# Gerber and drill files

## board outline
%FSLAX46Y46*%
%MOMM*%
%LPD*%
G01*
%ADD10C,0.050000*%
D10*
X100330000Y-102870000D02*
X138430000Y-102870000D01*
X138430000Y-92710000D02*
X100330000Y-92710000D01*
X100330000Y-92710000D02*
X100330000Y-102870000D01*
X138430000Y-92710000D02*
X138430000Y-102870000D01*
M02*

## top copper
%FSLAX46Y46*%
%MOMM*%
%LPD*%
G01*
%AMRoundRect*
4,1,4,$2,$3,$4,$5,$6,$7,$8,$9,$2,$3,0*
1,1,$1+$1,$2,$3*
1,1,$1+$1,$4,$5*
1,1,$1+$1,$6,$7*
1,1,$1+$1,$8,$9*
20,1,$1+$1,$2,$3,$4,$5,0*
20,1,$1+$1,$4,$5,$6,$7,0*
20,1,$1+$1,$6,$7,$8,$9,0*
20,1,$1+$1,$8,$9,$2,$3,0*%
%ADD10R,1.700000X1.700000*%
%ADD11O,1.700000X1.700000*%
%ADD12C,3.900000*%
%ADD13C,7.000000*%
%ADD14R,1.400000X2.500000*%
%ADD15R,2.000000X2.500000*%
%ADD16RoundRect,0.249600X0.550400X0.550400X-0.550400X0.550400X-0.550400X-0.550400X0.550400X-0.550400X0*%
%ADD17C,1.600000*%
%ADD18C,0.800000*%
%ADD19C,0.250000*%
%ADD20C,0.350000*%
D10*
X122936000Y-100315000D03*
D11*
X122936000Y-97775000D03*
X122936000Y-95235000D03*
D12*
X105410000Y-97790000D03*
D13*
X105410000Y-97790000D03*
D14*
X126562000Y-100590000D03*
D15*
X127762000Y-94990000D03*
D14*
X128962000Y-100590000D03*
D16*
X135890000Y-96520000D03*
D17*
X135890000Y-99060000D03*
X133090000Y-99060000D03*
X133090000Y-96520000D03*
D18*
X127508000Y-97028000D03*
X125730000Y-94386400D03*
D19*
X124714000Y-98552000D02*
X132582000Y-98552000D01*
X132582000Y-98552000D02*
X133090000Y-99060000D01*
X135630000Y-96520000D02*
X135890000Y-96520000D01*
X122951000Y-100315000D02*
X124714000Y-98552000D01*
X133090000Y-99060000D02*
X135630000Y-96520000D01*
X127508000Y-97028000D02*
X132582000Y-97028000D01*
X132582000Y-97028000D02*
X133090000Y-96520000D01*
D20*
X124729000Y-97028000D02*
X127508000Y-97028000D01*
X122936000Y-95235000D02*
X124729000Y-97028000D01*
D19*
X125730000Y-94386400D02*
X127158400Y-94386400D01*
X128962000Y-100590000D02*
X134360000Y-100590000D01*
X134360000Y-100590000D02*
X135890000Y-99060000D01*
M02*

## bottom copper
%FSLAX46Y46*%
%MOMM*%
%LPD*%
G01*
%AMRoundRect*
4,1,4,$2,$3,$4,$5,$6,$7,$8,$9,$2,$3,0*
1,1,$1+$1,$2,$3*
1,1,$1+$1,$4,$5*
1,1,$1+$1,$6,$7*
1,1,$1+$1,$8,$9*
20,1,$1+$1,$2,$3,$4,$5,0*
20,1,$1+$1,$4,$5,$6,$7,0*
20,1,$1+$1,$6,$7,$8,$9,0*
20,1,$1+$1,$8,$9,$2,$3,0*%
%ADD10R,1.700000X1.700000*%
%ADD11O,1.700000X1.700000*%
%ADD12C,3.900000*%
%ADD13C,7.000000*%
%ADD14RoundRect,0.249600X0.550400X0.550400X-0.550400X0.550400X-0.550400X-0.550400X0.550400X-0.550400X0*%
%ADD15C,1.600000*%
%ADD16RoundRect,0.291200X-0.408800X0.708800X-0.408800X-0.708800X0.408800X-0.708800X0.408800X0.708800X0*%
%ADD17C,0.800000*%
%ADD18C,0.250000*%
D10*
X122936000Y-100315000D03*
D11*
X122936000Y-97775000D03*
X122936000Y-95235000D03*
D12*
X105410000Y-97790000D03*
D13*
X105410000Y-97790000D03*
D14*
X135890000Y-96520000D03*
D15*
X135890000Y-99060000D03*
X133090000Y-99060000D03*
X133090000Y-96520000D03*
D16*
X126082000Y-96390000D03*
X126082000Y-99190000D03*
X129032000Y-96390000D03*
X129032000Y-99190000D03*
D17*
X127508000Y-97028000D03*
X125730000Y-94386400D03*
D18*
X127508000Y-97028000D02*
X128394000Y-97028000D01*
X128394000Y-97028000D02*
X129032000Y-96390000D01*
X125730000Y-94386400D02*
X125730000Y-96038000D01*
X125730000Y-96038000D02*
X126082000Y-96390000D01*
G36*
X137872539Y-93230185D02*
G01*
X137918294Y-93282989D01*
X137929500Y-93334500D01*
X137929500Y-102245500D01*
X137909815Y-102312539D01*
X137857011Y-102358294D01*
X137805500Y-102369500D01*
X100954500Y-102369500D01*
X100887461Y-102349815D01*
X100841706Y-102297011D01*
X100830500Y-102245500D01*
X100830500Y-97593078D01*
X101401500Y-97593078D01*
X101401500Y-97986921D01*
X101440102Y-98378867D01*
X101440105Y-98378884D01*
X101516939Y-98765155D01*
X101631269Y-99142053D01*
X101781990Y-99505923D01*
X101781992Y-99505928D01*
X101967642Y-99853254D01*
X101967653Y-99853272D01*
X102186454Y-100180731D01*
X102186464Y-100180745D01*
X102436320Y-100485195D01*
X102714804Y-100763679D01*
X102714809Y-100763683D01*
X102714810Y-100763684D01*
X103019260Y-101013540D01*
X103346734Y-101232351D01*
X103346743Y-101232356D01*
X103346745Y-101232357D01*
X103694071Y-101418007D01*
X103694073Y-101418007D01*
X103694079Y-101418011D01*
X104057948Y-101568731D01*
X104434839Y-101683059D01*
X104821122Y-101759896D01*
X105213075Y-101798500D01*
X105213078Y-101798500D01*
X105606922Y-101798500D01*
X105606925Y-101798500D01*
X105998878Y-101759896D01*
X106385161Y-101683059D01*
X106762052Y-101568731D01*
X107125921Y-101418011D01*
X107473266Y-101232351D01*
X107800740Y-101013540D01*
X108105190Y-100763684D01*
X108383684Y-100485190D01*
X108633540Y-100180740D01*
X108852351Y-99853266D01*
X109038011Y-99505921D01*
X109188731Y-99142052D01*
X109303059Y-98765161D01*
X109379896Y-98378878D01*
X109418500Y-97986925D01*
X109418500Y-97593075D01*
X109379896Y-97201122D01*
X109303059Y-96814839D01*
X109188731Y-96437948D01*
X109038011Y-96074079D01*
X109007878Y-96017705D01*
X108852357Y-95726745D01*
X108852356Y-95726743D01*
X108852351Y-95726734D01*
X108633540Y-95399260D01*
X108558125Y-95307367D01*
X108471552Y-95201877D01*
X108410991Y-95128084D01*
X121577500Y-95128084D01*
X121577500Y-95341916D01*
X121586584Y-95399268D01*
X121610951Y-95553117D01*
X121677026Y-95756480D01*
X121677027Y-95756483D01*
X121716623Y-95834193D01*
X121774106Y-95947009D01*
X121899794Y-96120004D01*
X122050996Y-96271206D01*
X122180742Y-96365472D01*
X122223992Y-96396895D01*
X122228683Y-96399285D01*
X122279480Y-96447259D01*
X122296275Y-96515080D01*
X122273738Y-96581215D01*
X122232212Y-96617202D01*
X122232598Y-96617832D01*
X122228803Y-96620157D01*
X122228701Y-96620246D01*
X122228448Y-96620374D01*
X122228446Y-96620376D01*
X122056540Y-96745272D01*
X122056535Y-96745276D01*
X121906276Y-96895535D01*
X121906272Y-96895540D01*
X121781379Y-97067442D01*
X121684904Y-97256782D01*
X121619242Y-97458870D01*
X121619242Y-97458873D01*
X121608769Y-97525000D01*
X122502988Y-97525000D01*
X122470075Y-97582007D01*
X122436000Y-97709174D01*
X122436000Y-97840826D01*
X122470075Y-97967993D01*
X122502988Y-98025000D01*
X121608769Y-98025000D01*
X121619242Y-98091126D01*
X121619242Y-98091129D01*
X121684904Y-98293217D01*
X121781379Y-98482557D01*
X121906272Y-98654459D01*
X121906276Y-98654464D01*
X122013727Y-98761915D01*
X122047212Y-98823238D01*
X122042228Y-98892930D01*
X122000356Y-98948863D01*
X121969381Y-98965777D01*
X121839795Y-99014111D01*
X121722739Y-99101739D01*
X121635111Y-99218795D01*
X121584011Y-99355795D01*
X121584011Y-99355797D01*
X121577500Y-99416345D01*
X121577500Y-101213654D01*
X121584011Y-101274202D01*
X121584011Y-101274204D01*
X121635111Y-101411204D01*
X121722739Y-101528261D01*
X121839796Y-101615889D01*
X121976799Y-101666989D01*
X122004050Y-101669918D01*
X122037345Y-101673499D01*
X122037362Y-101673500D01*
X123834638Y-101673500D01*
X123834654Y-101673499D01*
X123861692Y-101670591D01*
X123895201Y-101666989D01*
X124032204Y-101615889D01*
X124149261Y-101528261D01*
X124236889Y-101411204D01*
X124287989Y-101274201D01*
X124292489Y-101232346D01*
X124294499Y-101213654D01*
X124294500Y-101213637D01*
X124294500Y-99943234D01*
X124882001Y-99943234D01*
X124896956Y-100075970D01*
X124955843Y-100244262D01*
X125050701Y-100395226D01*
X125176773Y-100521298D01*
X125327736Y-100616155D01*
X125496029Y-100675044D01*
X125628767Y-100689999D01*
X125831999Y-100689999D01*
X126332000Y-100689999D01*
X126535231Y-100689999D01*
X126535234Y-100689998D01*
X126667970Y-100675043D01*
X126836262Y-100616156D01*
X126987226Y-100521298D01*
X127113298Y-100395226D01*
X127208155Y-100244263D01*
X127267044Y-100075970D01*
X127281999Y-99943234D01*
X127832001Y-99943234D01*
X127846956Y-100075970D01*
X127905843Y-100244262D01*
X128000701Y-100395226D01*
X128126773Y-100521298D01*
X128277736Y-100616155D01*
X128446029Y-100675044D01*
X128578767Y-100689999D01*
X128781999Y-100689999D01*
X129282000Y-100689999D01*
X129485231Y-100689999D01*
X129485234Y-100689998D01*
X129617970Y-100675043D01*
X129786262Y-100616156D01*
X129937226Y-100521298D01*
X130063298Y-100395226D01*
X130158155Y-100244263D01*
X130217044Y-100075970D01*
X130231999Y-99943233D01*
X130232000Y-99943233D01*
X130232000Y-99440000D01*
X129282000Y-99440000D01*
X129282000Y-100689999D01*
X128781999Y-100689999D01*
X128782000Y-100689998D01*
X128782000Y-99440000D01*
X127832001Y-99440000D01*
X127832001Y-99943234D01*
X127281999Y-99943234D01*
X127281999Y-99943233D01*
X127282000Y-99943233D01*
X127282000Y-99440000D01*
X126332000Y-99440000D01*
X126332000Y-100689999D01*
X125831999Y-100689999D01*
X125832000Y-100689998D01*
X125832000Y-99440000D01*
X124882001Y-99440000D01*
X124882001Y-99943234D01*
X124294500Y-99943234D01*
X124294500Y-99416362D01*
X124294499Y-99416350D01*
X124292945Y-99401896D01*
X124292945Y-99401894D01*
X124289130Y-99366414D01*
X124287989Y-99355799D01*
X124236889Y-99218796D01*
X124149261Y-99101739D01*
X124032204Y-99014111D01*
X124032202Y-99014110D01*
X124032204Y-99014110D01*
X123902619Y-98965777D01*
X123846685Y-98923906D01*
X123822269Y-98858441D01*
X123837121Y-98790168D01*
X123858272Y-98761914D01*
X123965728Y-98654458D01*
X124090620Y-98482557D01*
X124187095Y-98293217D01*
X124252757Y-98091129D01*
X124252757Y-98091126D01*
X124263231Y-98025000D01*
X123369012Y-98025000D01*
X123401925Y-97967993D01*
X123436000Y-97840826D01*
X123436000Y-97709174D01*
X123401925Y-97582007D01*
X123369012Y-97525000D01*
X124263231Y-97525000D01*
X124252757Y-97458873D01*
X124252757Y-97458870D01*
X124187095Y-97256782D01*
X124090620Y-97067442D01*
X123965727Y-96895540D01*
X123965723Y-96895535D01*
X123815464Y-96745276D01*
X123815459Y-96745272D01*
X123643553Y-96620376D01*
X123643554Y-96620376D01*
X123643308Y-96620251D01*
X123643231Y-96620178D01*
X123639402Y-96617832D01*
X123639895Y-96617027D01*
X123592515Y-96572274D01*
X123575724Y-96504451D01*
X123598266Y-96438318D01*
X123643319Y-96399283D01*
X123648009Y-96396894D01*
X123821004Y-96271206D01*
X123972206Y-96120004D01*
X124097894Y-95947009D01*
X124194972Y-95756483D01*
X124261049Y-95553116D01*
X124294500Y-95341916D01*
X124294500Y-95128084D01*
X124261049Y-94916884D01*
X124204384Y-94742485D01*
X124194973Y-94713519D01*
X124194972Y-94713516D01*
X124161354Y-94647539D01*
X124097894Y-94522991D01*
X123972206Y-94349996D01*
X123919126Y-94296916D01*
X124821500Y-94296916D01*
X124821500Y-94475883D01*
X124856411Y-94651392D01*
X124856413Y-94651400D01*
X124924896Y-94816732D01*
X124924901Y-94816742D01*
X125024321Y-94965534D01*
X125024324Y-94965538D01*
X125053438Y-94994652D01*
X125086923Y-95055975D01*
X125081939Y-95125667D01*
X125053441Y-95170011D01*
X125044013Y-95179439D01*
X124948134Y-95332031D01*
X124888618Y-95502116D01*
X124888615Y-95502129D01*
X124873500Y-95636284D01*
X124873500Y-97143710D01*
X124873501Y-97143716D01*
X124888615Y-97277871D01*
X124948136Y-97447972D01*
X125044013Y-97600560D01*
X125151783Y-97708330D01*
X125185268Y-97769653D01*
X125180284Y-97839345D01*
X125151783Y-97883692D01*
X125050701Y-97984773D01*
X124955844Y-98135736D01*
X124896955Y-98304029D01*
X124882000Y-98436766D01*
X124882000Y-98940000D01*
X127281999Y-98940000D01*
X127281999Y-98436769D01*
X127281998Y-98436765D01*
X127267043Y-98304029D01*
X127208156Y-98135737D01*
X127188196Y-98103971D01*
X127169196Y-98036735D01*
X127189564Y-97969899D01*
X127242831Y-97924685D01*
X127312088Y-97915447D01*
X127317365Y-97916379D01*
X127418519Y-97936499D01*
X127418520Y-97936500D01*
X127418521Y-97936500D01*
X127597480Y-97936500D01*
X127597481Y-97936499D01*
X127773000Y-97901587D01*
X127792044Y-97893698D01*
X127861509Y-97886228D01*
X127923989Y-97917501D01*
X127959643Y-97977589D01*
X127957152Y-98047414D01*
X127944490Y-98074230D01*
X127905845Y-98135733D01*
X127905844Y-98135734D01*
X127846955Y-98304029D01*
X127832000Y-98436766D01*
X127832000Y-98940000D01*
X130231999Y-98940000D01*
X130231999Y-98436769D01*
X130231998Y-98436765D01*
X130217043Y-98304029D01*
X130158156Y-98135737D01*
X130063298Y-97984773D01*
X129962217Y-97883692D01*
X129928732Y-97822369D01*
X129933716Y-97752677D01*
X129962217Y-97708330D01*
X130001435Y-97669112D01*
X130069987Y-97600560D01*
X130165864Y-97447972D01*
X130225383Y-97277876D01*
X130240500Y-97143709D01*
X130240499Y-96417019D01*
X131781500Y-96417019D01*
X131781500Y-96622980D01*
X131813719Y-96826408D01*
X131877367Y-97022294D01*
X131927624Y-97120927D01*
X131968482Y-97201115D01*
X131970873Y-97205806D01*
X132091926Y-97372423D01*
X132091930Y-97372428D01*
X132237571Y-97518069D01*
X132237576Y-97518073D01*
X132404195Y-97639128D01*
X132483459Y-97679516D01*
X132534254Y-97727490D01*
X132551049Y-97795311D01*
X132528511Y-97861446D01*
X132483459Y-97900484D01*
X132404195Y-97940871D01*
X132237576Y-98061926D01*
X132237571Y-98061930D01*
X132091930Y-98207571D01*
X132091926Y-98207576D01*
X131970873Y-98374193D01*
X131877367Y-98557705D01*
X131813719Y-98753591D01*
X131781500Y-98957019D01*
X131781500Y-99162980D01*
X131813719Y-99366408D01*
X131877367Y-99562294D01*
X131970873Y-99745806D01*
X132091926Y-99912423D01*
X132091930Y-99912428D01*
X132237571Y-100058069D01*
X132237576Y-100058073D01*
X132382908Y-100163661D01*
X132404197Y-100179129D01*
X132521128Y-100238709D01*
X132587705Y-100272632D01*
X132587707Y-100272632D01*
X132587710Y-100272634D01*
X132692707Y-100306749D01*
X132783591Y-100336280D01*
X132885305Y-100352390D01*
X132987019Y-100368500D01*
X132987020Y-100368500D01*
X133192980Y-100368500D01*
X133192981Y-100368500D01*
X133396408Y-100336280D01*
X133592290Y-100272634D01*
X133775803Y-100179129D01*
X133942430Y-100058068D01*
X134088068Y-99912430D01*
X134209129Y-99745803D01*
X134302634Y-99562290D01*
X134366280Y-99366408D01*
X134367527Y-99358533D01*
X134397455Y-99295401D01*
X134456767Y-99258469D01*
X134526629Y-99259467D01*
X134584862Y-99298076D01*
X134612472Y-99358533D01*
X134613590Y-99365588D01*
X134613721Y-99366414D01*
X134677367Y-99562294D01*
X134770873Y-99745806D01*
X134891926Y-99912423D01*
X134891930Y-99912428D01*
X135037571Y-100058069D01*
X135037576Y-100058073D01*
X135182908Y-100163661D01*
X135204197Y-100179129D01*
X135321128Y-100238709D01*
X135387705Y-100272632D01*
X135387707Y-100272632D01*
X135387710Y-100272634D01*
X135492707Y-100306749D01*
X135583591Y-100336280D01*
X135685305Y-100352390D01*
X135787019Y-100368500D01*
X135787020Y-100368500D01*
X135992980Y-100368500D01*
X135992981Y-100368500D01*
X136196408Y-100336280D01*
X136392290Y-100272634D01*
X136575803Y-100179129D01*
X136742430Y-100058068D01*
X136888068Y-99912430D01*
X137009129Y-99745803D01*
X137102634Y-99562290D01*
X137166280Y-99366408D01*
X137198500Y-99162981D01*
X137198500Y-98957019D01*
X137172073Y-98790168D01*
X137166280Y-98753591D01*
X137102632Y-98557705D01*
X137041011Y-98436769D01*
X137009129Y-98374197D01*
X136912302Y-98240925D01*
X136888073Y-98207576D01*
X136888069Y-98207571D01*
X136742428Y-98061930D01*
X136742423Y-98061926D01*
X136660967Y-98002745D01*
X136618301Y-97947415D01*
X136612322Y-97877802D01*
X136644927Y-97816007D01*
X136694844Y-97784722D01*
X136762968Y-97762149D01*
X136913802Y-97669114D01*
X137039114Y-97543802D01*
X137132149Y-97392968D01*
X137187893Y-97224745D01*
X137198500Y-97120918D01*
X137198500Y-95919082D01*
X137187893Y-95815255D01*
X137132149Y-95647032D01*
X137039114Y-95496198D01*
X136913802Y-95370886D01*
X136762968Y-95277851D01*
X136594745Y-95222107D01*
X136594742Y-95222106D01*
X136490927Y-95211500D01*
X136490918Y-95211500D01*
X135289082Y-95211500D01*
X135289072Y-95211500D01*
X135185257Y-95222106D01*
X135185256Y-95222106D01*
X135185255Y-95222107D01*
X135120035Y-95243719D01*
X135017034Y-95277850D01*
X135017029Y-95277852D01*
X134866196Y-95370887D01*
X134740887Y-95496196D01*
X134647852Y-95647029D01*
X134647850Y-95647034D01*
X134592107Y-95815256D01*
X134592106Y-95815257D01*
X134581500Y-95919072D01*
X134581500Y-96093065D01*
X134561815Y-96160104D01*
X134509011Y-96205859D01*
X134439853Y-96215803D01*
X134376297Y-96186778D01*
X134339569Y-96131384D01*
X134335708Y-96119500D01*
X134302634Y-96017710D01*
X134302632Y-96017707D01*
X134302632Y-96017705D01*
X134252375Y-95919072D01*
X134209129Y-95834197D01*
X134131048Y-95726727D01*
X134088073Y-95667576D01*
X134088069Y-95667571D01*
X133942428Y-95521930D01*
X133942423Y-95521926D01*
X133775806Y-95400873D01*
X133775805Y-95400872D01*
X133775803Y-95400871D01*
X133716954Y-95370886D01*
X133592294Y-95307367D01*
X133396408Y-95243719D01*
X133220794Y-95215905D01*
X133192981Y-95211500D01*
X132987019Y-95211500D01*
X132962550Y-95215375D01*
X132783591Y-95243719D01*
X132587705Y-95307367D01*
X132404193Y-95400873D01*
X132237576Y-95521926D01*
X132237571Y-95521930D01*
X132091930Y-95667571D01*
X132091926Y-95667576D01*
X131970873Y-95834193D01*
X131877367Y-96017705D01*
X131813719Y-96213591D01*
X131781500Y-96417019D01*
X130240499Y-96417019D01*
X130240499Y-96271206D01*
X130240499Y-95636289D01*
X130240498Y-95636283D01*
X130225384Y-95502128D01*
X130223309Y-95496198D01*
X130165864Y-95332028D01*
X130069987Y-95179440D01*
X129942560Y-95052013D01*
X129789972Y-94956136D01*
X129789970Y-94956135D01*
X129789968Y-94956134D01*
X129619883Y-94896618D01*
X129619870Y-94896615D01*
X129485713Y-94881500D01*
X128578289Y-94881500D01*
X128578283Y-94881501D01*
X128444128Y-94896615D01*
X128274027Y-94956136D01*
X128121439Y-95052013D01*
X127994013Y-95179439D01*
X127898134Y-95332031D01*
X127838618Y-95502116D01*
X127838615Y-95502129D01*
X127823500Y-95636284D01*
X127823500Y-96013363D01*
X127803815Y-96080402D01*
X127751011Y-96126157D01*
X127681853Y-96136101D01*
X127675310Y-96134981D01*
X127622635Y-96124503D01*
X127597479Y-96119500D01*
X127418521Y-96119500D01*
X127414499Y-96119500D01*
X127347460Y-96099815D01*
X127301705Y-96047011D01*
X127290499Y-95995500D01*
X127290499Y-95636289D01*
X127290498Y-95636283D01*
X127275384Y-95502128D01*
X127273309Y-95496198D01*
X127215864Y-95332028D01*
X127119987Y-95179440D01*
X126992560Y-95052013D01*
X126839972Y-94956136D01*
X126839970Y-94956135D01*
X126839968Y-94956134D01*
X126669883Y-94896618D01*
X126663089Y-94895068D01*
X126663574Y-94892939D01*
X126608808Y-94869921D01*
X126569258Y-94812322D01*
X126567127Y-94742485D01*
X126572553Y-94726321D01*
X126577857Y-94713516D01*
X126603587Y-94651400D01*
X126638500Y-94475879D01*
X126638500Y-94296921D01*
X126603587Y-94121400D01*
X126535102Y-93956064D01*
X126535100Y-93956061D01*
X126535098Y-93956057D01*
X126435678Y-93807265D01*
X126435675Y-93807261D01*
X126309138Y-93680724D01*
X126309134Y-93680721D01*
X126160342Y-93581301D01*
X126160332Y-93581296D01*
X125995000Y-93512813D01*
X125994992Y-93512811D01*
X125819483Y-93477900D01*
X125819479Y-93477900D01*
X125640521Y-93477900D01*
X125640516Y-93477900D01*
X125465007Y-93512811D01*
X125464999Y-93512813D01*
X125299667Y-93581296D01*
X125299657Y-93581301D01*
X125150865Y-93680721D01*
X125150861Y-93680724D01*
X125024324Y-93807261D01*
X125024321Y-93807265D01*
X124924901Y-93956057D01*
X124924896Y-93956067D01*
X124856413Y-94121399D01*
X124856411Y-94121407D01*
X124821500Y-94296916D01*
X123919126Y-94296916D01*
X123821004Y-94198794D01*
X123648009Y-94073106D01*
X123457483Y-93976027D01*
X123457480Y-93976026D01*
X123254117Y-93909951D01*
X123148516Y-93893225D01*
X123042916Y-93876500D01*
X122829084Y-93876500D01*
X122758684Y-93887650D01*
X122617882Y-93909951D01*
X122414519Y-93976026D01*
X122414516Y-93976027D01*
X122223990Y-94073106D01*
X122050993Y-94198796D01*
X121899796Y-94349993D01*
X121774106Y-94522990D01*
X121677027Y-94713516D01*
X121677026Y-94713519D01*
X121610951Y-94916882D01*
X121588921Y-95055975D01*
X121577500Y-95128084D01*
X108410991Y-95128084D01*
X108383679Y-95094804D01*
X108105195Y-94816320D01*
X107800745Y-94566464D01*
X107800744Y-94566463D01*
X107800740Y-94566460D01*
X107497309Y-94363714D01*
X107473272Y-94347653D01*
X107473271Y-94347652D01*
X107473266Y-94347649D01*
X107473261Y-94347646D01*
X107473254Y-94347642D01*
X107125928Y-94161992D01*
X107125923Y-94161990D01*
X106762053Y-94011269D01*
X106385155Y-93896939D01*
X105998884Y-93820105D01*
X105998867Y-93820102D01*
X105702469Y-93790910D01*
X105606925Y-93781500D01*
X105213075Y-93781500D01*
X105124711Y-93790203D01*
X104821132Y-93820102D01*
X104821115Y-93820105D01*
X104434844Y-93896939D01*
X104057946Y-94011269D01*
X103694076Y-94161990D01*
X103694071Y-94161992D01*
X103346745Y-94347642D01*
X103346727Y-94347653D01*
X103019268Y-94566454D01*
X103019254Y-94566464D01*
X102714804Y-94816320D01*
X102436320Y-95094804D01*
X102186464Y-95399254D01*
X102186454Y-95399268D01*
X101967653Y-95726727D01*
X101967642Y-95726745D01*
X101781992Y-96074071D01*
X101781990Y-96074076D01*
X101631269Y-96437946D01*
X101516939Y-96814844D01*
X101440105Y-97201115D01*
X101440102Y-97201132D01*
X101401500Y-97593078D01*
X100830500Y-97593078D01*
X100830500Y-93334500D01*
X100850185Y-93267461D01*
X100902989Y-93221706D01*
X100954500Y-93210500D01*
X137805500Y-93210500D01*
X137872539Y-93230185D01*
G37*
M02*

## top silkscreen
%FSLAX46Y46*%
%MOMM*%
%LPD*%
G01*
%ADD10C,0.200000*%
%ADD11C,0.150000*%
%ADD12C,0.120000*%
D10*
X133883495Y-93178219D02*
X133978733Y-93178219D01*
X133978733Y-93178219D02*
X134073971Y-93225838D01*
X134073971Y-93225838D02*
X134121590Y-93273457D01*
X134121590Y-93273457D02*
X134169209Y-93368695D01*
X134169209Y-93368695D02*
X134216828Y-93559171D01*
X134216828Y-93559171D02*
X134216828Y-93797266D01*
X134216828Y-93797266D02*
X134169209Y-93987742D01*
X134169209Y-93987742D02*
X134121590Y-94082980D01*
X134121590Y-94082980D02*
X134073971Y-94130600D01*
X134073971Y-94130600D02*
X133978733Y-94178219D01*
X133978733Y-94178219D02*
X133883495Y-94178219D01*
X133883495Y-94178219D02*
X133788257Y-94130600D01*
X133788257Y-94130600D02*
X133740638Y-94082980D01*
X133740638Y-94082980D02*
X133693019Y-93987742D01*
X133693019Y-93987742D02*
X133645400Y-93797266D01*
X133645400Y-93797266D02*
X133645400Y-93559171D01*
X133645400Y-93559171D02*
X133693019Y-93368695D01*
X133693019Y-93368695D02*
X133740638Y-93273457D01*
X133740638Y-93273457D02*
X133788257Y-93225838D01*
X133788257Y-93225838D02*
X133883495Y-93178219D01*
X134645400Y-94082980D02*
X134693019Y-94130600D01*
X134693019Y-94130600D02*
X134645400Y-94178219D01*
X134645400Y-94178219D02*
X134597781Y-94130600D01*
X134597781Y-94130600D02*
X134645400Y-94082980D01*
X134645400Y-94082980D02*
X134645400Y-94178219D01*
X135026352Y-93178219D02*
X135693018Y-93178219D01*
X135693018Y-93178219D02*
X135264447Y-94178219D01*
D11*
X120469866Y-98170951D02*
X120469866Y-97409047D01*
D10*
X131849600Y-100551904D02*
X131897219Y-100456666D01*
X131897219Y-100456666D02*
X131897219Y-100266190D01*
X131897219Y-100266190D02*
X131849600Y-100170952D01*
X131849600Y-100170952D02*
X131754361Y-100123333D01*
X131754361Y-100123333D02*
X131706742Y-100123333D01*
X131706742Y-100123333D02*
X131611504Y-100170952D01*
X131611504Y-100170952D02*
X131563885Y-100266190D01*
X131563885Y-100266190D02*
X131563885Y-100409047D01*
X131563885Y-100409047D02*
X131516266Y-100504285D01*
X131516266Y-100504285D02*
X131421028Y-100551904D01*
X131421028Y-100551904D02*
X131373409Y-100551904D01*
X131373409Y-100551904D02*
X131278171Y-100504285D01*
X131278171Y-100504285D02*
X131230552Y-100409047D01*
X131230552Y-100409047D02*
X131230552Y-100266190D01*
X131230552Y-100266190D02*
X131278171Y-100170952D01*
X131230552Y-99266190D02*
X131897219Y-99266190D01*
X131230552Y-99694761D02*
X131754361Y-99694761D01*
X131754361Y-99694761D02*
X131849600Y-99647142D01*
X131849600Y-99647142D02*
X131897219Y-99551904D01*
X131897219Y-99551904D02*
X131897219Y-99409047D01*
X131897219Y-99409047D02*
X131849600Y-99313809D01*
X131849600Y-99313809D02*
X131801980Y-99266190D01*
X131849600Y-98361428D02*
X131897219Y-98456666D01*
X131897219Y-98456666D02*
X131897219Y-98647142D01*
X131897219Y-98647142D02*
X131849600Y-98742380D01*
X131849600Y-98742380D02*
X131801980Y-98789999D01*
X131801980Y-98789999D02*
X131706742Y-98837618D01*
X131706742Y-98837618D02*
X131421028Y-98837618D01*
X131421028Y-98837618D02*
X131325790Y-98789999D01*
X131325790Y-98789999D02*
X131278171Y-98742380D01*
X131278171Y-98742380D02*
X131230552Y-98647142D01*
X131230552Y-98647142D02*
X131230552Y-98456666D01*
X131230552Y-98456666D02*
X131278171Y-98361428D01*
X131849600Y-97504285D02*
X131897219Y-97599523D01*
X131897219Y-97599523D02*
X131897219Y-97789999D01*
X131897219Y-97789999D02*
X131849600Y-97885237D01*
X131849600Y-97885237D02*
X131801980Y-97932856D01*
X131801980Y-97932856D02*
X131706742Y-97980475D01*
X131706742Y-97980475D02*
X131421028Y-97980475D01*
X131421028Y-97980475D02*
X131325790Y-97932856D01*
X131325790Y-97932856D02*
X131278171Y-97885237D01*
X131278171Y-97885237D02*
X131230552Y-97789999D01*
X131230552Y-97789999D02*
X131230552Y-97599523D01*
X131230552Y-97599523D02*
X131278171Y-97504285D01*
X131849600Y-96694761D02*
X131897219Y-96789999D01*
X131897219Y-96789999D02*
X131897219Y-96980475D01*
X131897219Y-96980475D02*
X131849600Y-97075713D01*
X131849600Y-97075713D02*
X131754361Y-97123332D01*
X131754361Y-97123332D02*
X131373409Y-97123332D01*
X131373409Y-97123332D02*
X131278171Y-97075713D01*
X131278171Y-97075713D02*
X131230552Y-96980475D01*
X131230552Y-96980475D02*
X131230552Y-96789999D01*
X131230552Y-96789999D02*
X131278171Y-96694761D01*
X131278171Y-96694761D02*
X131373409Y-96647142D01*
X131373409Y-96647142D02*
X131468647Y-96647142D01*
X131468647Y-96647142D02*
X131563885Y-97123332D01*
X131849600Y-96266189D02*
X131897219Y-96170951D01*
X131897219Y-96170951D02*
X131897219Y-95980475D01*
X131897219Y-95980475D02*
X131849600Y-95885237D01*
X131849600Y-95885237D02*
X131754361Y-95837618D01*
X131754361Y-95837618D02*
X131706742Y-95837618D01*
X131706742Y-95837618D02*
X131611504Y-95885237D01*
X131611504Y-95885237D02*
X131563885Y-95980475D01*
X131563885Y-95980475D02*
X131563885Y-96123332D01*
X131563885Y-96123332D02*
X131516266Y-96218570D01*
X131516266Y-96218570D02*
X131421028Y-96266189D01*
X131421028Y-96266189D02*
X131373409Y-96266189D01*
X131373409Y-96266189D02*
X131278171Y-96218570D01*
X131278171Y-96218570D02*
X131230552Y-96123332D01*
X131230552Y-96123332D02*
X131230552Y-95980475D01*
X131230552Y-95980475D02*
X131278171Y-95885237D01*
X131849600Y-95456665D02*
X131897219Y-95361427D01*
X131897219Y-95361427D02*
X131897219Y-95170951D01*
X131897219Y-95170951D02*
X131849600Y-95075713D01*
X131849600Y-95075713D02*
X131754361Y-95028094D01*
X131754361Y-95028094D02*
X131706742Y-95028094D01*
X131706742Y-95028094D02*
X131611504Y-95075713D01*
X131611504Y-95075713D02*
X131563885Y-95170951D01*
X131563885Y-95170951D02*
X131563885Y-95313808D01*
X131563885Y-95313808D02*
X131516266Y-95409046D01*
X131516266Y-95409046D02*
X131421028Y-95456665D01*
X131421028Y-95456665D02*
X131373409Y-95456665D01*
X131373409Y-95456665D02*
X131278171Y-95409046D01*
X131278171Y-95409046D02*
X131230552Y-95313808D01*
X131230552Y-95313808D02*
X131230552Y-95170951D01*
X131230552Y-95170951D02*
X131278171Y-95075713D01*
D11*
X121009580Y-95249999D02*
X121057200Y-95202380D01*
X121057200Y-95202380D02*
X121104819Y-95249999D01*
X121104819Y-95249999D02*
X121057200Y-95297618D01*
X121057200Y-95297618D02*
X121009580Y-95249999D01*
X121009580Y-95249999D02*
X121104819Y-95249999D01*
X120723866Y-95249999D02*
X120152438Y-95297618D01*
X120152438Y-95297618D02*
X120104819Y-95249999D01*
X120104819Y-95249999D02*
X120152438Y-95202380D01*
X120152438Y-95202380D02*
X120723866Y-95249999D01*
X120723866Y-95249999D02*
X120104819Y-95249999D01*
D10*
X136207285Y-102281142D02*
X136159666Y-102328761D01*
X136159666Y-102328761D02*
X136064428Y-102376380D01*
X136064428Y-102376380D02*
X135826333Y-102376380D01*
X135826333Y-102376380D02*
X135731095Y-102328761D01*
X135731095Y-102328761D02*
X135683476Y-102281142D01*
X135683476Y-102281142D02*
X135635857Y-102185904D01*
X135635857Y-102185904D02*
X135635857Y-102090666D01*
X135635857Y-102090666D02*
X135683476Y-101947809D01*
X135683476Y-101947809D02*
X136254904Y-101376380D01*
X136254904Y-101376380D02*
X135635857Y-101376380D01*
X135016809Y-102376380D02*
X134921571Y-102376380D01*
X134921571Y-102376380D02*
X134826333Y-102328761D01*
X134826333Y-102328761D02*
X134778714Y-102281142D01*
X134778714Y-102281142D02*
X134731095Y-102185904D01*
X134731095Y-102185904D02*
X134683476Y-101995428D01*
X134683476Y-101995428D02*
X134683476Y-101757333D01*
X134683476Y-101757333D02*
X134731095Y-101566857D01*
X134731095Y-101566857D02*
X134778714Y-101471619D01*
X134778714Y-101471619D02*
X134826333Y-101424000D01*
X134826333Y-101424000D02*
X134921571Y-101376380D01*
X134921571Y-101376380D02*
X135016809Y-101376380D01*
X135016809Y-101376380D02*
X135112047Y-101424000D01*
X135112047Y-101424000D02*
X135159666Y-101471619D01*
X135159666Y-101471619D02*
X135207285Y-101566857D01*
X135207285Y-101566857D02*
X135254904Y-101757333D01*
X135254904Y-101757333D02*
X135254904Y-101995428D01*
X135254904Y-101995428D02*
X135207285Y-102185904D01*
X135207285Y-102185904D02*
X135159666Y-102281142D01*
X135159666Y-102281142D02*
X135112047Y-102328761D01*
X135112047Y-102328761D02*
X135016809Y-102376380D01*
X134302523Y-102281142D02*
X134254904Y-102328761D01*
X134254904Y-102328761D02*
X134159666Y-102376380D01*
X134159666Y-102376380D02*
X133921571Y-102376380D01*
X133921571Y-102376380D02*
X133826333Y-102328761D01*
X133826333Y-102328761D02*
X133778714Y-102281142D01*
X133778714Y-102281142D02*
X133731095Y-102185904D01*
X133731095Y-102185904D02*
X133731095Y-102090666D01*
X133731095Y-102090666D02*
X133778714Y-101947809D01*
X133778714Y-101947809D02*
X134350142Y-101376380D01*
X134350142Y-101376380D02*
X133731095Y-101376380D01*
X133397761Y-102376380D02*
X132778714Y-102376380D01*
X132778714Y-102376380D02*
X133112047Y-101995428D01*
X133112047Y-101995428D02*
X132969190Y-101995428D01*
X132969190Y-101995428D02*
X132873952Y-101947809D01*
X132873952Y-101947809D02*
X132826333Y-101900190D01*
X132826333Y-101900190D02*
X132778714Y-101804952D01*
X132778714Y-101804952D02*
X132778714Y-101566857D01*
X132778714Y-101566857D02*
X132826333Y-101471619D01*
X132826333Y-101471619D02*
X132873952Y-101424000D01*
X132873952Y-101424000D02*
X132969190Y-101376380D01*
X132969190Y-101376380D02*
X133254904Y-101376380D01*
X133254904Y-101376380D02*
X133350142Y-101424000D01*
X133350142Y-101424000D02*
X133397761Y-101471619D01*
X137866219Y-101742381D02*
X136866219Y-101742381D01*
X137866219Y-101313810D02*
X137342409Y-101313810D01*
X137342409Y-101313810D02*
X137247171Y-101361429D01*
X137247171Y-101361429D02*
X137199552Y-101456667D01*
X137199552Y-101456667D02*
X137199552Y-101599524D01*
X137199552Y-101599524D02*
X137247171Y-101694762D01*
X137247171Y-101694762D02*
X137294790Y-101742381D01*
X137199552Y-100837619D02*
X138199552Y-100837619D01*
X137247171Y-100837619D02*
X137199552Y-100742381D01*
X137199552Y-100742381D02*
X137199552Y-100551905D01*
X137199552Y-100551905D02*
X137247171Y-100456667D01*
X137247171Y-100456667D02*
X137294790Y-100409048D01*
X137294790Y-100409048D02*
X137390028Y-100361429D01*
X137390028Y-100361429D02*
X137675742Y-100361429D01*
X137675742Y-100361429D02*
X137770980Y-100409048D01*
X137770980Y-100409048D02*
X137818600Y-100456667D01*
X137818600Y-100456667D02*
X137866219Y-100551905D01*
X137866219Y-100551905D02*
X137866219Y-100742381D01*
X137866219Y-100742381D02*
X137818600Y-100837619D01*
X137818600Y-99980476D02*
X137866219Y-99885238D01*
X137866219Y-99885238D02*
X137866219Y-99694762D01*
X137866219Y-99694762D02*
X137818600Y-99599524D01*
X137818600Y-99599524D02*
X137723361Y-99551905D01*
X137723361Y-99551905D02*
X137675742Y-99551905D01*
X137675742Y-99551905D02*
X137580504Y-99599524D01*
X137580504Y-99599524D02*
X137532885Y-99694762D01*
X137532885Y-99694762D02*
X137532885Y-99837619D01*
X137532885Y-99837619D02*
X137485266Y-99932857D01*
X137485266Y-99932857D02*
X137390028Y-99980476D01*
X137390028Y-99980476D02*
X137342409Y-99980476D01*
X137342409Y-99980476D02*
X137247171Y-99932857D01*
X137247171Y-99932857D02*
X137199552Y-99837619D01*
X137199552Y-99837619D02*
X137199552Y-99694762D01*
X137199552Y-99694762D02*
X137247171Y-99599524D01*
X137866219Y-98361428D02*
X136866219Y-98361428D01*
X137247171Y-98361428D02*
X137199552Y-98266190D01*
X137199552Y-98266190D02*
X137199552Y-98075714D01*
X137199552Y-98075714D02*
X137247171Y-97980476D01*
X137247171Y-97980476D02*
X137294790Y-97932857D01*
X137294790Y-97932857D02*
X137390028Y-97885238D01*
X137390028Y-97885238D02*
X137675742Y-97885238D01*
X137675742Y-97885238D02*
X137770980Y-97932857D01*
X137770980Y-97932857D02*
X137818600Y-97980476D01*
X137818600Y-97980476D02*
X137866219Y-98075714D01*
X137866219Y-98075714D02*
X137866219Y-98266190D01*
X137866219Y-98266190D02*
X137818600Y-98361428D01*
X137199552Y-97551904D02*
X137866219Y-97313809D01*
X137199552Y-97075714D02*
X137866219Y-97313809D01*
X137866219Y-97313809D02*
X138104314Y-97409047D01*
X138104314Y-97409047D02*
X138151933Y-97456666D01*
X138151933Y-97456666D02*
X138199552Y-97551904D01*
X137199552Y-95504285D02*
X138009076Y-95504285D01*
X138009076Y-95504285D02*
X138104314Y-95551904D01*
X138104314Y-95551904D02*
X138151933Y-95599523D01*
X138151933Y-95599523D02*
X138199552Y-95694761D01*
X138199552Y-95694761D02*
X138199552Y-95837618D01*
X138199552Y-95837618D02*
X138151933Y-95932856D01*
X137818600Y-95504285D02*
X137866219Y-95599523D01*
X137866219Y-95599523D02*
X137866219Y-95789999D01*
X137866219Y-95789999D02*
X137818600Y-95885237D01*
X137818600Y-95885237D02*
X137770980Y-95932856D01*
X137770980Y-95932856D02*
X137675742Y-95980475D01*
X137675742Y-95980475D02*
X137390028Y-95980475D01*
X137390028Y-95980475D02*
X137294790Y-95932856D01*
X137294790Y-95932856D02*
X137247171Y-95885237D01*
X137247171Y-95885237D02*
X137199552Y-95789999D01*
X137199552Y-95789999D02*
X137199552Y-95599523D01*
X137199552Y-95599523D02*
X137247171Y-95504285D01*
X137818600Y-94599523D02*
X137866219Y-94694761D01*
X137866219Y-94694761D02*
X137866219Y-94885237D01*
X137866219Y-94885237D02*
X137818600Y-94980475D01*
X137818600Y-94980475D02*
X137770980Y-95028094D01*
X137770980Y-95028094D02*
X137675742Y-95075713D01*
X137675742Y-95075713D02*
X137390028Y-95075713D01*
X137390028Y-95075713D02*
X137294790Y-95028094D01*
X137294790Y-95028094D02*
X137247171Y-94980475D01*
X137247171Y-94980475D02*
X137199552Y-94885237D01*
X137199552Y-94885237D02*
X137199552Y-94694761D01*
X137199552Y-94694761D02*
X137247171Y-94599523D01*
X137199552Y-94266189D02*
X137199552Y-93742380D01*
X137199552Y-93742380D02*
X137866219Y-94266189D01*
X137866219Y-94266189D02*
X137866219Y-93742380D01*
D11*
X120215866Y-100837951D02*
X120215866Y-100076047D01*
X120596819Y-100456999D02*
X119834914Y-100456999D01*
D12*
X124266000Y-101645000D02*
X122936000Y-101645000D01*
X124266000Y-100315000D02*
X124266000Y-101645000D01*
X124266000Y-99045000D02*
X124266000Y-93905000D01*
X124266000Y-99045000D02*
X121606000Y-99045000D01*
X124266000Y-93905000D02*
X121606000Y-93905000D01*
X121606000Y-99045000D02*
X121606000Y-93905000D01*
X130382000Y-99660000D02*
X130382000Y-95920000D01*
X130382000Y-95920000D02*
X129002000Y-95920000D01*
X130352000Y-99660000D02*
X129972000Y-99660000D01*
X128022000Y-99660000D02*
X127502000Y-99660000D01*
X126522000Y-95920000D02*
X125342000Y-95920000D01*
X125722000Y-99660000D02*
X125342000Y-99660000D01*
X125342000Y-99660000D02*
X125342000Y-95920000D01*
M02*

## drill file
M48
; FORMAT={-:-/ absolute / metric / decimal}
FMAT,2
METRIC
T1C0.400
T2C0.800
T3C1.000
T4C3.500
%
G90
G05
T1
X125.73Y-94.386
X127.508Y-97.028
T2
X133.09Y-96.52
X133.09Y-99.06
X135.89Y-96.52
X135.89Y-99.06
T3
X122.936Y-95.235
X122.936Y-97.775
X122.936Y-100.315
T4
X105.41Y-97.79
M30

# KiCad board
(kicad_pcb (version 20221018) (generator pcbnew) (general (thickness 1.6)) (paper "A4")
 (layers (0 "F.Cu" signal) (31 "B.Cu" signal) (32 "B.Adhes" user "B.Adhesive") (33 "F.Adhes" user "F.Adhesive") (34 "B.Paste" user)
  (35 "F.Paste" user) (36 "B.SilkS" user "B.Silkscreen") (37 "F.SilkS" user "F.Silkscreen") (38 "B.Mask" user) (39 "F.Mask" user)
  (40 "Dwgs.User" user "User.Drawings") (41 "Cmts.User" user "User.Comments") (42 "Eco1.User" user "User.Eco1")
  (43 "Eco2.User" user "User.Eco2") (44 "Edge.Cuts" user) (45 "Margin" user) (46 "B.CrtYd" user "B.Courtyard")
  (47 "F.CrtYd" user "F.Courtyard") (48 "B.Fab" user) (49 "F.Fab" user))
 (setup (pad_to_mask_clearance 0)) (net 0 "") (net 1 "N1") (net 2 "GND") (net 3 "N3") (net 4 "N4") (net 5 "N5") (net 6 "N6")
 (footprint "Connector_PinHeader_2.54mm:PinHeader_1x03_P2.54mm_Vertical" (layer "F.Cu") (at 122.936 100.315 180)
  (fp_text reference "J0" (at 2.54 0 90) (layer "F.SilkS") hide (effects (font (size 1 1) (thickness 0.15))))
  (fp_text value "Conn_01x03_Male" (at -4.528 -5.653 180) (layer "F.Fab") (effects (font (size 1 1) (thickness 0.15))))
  (fp_line (start -1.33 -1.33) (end 0 -1.33) (stroke (width 0.12) (type solid)) (layer "F.SilkS"))
  (fp_line (start -1.33 0) (end -1.33 -1.33) (stroke (width 0.12) (type solid)) (layer "F.SilkS"))
  (fp_line (start -1.33 1.27) (end -1.33 6.41) (stroke (width 0.12) (type solid)) (layer "F.SilkS"))
  (fp_line (start -1.33 1.27) (end 1.33 1.27) (stroke (width 0.12) (type solid)) (layer "F.SilkS"))
  (fp_line (start -1.33 6.41) (end 1.33 6.41) (stroke (width 0.12) (type solid)) (layer "F.SilkS"))
  (fp_line (start 1.33 1.27) (end 1.33 6.41) (stroke (width 0.12) (type solid)) (layer "F.SilkS"))
  (pad "1" thru_hole rect (at 0 0 180) (size 1.7 1.7) (drill 1) (layers "*.Cu" "*.Mask") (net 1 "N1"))
  (pad "2" thru_hole oval (at 0 2.54 180) (size 1.7 1.7) (drill 1) (layers "*.Cu" "*.Mask") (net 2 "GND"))
  (pad "3" thru_hole oval (at 0 5.08 180) (size 1.7 1.7) (drill 1) (layers "*.Cu" "*.Mask") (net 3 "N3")))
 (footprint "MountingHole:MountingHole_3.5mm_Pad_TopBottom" (layer "F.Cu") (at 105.41 97.79)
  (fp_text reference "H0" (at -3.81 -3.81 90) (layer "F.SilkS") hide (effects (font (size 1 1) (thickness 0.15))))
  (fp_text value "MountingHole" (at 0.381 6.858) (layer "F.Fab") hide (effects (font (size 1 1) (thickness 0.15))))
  (pad "1" thru_hole circle (at 0 0) (size 3.9 3.9) (drill 3.5) (layers "*.Cu" "*.Mask"))
  (pad "1" connect circle (at 0 0) (size 7 7) (layers "F.Cu" "F.Mask"))
  (pad "1" connect circle (at 0 0) (size 7 7) (layers "B.Cu" "B.Mask")))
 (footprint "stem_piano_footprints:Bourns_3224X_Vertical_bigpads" (layer "F.Cu") (at 127.762 97.79 180)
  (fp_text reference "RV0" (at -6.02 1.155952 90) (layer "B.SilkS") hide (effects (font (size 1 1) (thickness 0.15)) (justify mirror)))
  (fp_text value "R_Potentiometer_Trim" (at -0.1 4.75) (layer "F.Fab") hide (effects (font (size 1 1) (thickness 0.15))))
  (fp_line (start -2.62 -1.87) (end -2.62 1.87) (stroke (width 0.12) (type solid)) (layer "F.SilkS"))
  (fp_line (start -2.62 1.87) (end -1.24 1.87) (stroke (width 0.12) (type solid)) (layer "F.SilkS"))
  (fp_line (start -2.59 -1.87) (end -2.21 -1.87) (stroke (width 0.12) (type solid)) (layer "F.SilkS"))
  (fp_line (start -0.26 -1.87) (end 0.26 -1.87) (stroke (width 0.12) (type solid)) (layer "F.SilkS"))
  (fp_line (start 1.24 1.87) (end 2.42 1.87) (stroke (width 0.12) (type solid)) (layer "F.SilkS"))
  (fp_line (start 2.04 -1.87) (end 2.42 -1.87) (stroke (width 0.12) (type solid)) (layer "F.SilkS"))
  (fp_line (start 2.42 -1.87) (end 2.42 1.87) (stroke (width 0.12) (type solid)) (layer "F.SilkS"))
  (pad "1" smd rect (at 1.2 -2.8 180) (size 1.4 2.5) (layers "F.Cu" "F.Paste" "F.Mask") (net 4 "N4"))
  (pad "2" smd rect (at 0 2.8 180) (size 2 2.5) (layers "F.Cu" "F.Paste" "F.Mask") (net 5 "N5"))
  (pad "3" smd rect (at -1.2 -2.8 180) (size 1.4 2.5) (layers "F.Cu" "F.Paste" "F.Mask") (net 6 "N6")))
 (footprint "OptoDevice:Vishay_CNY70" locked (layer "B.Cu") (at 135.89 96.52 180)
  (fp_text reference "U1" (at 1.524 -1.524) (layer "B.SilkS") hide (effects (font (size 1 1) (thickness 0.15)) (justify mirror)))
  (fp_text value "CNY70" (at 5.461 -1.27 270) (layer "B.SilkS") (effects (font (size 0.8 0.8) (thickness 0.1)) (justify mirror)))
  (pad "1" thru_hole roundrect locked (at 0 0 180) (size 1.6 1.6) (drill 0.8) (layers "*.Cu" "*.Mask") (roundrect_rratio 0.156) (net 1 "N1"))
  (pad "2" thru_hole circle locked (at 0 -2.54 180) (size 1.6 1.6) (drill 0.8) (layers "*.Cu" "*.Mask") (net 6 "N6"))
  (pad "3" thru_hole circle locked (at 2.8 -2.54 180) (size 1.6 1.6) (drill 0.8) (layers "*.Cu" "*.Mask") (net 1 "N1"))
  (pad "4" thru_hole circle locked (at 2.8 0 180) (size 1.6 1.6) (drill 0.8) (layers "*.Cu" "*.Mask") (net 3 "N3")))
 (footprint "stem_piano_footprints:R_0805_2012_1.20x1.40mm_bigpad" (layer "B.Cu") (at 126.082 97.79 -90)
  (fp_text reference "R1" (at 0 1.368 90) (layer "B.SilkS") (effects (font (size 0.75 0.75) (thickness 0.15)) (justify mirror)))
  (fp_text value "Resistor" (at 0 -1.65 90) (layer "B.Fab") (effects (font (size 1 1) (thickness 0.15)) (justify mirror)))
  (pad "1" smd roundrect (at -1.4 0 270) (size 2 1.4) (layers "B.Cu" "B.Paste" "B.Mask") (roundrect_rratio 0.208) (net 5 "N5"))
  (pad "2" smd roundrect (at 1.4 0 270) (size 2 1.4) (layers "B.Cu" "B.Paste" "B.Mask") (roundrect_rratio 0.208) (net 2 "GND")))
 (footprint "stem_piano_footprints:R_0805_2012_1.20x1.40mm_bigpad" (layer "B.Cu") (at 129.032 97.79 -90)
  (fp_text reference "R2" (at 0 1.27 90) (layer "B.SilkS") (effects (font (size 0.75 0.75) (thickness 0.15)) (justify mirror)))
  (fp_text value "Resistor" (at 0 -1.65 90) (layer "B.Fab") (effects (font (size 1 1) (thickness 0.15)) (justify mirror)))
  (pad "1" smd roundrect (at -1.4 0 270) (size 2 1.4) (layers "B.Cu" "B.Paste" "B.Mask") (roundrect_rratio 0.208) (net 3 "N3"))
  (pad "2" smd roundrect (at 1.4 0 270) (size 2 1.4) (layers "B.Cu" "B.Paste" "B.Mask") (roundrect_rratio 0.208) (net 2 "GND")))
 (gr_line (start 100.33 102.87) (end 138.43 102.87) (stroke (width 0.05) (type solid)) (layer "Edge.Cuts"))
 (gr_line (start 138.43 92.71) (end 100.33 92.71) (stroke (width 0.05) (type solid)) (layer "Edge.Cuts"))
 (gr_line (start 100.33 92.71) (end 100.33 102.87) (stroke (width 0.05) (type solid)) (layer "Edge.Cuts"))
 (gr_line (start 138.43 92.71) (end 138.43 102.87) (stroke (width 0.05) (type solid)) (layer "Edge.Cuts"))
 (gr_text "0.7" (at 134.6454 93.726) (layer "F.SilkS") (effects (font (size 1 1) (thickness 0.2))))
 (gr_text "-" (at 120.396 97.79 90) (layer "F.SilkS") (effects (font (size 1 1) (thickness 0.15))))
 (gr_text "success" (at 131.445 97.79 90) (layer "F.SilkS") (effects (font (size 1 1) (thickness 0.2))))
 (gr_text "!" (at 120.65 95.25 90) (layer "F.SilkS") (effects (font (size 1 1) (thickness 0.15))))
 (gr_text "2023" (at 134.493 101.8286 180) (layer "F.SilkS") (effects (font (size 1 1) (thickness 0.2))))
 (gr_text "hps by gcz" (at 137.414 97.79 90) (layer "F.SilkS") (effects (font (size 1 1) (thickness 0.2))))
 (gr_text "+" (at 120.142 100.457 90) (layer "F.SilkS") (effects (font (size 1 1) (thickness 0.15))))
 (segment (start 124.714 98.552) (end 132.582 98.552) (width 0.25) (layer "F.Cu") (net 1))
 (segment (start 132.582 98.552) (end 133.09 99.06) (width 0.25) (layer "F.Cu") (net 1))
 (segment (start 135.63 96.52) (end 135.89 96.52) (width 0.25) (layer "F.Cu") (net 1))
 (segment (start 122.951 100.315) (end 124.714 98.552) (width 0.25) (layer "F.Cu") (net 1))
 (segment (start 133.09 99.06) (end 135.63 96.52) (width 0.25) (layer "F.Cu") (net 1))
 (segment (start 127.508 97.028) (end 132.582 97.028) (width 0.25) (layer "F.Cu") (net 3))
 (segment (start 132.582 97.028) (end 133.09 96.52) (width 0.25) (layer "F.Cu") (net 3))
 (segment (start 124.729 97.028) (end 127.508 97.028) (width 0.35) (layer "F.Cu") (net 3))
 (segment (start 122.936 95.235) (end 124.729 97.028) (width 0.35) (layer "F.Cu") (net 3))
 (via (at 127.508 97.028) (size 0.8) (drill 0.4) (layers "F.Cu" "B.Cu") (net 3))
 (segment (start 127.508 97.028) (end 128.394 97.028) (width 0.25) (layer "B.Cu") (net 3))
 (segment (start 128.394 97.028) (end 129.032 96.39) (width 0.25) (layer "B.Cu") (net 3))
 (segment (start 125.73 94.3864) (end 127.1584 94.3864) (width 0.25) (layer "F.Cu") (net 5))
 (via (at 125.73 94.3864) (size 0.8) (drill 0.4) (layers "F.Cu" "B.Cu") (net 5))
 (segment (start 125.73 94.3864) (end 125.73 96.038) (width 0.25) (layer "B.Cu") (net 5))
 (segment (start 125.73 96.038) (end 126.082 96.39) (width 0.25) (layer "B.Cu") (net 5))
 (segment (start 128.962 100.59) (end 134.36 100.59) (width 0.25) (layer "F.Cu") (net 6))
 (segment (start 134.36 100.59) (end 135.89 99.06) (width 0.25) (layer "F.Cu") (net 6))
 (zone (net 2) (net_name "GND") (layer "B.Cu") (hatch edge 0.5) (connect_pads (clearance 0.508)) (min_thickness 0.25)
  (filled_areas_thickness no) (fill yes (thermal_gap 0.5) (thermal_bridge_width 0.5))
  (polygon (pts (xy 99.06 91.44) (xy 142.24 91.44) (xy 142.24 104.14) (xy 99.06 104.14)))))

